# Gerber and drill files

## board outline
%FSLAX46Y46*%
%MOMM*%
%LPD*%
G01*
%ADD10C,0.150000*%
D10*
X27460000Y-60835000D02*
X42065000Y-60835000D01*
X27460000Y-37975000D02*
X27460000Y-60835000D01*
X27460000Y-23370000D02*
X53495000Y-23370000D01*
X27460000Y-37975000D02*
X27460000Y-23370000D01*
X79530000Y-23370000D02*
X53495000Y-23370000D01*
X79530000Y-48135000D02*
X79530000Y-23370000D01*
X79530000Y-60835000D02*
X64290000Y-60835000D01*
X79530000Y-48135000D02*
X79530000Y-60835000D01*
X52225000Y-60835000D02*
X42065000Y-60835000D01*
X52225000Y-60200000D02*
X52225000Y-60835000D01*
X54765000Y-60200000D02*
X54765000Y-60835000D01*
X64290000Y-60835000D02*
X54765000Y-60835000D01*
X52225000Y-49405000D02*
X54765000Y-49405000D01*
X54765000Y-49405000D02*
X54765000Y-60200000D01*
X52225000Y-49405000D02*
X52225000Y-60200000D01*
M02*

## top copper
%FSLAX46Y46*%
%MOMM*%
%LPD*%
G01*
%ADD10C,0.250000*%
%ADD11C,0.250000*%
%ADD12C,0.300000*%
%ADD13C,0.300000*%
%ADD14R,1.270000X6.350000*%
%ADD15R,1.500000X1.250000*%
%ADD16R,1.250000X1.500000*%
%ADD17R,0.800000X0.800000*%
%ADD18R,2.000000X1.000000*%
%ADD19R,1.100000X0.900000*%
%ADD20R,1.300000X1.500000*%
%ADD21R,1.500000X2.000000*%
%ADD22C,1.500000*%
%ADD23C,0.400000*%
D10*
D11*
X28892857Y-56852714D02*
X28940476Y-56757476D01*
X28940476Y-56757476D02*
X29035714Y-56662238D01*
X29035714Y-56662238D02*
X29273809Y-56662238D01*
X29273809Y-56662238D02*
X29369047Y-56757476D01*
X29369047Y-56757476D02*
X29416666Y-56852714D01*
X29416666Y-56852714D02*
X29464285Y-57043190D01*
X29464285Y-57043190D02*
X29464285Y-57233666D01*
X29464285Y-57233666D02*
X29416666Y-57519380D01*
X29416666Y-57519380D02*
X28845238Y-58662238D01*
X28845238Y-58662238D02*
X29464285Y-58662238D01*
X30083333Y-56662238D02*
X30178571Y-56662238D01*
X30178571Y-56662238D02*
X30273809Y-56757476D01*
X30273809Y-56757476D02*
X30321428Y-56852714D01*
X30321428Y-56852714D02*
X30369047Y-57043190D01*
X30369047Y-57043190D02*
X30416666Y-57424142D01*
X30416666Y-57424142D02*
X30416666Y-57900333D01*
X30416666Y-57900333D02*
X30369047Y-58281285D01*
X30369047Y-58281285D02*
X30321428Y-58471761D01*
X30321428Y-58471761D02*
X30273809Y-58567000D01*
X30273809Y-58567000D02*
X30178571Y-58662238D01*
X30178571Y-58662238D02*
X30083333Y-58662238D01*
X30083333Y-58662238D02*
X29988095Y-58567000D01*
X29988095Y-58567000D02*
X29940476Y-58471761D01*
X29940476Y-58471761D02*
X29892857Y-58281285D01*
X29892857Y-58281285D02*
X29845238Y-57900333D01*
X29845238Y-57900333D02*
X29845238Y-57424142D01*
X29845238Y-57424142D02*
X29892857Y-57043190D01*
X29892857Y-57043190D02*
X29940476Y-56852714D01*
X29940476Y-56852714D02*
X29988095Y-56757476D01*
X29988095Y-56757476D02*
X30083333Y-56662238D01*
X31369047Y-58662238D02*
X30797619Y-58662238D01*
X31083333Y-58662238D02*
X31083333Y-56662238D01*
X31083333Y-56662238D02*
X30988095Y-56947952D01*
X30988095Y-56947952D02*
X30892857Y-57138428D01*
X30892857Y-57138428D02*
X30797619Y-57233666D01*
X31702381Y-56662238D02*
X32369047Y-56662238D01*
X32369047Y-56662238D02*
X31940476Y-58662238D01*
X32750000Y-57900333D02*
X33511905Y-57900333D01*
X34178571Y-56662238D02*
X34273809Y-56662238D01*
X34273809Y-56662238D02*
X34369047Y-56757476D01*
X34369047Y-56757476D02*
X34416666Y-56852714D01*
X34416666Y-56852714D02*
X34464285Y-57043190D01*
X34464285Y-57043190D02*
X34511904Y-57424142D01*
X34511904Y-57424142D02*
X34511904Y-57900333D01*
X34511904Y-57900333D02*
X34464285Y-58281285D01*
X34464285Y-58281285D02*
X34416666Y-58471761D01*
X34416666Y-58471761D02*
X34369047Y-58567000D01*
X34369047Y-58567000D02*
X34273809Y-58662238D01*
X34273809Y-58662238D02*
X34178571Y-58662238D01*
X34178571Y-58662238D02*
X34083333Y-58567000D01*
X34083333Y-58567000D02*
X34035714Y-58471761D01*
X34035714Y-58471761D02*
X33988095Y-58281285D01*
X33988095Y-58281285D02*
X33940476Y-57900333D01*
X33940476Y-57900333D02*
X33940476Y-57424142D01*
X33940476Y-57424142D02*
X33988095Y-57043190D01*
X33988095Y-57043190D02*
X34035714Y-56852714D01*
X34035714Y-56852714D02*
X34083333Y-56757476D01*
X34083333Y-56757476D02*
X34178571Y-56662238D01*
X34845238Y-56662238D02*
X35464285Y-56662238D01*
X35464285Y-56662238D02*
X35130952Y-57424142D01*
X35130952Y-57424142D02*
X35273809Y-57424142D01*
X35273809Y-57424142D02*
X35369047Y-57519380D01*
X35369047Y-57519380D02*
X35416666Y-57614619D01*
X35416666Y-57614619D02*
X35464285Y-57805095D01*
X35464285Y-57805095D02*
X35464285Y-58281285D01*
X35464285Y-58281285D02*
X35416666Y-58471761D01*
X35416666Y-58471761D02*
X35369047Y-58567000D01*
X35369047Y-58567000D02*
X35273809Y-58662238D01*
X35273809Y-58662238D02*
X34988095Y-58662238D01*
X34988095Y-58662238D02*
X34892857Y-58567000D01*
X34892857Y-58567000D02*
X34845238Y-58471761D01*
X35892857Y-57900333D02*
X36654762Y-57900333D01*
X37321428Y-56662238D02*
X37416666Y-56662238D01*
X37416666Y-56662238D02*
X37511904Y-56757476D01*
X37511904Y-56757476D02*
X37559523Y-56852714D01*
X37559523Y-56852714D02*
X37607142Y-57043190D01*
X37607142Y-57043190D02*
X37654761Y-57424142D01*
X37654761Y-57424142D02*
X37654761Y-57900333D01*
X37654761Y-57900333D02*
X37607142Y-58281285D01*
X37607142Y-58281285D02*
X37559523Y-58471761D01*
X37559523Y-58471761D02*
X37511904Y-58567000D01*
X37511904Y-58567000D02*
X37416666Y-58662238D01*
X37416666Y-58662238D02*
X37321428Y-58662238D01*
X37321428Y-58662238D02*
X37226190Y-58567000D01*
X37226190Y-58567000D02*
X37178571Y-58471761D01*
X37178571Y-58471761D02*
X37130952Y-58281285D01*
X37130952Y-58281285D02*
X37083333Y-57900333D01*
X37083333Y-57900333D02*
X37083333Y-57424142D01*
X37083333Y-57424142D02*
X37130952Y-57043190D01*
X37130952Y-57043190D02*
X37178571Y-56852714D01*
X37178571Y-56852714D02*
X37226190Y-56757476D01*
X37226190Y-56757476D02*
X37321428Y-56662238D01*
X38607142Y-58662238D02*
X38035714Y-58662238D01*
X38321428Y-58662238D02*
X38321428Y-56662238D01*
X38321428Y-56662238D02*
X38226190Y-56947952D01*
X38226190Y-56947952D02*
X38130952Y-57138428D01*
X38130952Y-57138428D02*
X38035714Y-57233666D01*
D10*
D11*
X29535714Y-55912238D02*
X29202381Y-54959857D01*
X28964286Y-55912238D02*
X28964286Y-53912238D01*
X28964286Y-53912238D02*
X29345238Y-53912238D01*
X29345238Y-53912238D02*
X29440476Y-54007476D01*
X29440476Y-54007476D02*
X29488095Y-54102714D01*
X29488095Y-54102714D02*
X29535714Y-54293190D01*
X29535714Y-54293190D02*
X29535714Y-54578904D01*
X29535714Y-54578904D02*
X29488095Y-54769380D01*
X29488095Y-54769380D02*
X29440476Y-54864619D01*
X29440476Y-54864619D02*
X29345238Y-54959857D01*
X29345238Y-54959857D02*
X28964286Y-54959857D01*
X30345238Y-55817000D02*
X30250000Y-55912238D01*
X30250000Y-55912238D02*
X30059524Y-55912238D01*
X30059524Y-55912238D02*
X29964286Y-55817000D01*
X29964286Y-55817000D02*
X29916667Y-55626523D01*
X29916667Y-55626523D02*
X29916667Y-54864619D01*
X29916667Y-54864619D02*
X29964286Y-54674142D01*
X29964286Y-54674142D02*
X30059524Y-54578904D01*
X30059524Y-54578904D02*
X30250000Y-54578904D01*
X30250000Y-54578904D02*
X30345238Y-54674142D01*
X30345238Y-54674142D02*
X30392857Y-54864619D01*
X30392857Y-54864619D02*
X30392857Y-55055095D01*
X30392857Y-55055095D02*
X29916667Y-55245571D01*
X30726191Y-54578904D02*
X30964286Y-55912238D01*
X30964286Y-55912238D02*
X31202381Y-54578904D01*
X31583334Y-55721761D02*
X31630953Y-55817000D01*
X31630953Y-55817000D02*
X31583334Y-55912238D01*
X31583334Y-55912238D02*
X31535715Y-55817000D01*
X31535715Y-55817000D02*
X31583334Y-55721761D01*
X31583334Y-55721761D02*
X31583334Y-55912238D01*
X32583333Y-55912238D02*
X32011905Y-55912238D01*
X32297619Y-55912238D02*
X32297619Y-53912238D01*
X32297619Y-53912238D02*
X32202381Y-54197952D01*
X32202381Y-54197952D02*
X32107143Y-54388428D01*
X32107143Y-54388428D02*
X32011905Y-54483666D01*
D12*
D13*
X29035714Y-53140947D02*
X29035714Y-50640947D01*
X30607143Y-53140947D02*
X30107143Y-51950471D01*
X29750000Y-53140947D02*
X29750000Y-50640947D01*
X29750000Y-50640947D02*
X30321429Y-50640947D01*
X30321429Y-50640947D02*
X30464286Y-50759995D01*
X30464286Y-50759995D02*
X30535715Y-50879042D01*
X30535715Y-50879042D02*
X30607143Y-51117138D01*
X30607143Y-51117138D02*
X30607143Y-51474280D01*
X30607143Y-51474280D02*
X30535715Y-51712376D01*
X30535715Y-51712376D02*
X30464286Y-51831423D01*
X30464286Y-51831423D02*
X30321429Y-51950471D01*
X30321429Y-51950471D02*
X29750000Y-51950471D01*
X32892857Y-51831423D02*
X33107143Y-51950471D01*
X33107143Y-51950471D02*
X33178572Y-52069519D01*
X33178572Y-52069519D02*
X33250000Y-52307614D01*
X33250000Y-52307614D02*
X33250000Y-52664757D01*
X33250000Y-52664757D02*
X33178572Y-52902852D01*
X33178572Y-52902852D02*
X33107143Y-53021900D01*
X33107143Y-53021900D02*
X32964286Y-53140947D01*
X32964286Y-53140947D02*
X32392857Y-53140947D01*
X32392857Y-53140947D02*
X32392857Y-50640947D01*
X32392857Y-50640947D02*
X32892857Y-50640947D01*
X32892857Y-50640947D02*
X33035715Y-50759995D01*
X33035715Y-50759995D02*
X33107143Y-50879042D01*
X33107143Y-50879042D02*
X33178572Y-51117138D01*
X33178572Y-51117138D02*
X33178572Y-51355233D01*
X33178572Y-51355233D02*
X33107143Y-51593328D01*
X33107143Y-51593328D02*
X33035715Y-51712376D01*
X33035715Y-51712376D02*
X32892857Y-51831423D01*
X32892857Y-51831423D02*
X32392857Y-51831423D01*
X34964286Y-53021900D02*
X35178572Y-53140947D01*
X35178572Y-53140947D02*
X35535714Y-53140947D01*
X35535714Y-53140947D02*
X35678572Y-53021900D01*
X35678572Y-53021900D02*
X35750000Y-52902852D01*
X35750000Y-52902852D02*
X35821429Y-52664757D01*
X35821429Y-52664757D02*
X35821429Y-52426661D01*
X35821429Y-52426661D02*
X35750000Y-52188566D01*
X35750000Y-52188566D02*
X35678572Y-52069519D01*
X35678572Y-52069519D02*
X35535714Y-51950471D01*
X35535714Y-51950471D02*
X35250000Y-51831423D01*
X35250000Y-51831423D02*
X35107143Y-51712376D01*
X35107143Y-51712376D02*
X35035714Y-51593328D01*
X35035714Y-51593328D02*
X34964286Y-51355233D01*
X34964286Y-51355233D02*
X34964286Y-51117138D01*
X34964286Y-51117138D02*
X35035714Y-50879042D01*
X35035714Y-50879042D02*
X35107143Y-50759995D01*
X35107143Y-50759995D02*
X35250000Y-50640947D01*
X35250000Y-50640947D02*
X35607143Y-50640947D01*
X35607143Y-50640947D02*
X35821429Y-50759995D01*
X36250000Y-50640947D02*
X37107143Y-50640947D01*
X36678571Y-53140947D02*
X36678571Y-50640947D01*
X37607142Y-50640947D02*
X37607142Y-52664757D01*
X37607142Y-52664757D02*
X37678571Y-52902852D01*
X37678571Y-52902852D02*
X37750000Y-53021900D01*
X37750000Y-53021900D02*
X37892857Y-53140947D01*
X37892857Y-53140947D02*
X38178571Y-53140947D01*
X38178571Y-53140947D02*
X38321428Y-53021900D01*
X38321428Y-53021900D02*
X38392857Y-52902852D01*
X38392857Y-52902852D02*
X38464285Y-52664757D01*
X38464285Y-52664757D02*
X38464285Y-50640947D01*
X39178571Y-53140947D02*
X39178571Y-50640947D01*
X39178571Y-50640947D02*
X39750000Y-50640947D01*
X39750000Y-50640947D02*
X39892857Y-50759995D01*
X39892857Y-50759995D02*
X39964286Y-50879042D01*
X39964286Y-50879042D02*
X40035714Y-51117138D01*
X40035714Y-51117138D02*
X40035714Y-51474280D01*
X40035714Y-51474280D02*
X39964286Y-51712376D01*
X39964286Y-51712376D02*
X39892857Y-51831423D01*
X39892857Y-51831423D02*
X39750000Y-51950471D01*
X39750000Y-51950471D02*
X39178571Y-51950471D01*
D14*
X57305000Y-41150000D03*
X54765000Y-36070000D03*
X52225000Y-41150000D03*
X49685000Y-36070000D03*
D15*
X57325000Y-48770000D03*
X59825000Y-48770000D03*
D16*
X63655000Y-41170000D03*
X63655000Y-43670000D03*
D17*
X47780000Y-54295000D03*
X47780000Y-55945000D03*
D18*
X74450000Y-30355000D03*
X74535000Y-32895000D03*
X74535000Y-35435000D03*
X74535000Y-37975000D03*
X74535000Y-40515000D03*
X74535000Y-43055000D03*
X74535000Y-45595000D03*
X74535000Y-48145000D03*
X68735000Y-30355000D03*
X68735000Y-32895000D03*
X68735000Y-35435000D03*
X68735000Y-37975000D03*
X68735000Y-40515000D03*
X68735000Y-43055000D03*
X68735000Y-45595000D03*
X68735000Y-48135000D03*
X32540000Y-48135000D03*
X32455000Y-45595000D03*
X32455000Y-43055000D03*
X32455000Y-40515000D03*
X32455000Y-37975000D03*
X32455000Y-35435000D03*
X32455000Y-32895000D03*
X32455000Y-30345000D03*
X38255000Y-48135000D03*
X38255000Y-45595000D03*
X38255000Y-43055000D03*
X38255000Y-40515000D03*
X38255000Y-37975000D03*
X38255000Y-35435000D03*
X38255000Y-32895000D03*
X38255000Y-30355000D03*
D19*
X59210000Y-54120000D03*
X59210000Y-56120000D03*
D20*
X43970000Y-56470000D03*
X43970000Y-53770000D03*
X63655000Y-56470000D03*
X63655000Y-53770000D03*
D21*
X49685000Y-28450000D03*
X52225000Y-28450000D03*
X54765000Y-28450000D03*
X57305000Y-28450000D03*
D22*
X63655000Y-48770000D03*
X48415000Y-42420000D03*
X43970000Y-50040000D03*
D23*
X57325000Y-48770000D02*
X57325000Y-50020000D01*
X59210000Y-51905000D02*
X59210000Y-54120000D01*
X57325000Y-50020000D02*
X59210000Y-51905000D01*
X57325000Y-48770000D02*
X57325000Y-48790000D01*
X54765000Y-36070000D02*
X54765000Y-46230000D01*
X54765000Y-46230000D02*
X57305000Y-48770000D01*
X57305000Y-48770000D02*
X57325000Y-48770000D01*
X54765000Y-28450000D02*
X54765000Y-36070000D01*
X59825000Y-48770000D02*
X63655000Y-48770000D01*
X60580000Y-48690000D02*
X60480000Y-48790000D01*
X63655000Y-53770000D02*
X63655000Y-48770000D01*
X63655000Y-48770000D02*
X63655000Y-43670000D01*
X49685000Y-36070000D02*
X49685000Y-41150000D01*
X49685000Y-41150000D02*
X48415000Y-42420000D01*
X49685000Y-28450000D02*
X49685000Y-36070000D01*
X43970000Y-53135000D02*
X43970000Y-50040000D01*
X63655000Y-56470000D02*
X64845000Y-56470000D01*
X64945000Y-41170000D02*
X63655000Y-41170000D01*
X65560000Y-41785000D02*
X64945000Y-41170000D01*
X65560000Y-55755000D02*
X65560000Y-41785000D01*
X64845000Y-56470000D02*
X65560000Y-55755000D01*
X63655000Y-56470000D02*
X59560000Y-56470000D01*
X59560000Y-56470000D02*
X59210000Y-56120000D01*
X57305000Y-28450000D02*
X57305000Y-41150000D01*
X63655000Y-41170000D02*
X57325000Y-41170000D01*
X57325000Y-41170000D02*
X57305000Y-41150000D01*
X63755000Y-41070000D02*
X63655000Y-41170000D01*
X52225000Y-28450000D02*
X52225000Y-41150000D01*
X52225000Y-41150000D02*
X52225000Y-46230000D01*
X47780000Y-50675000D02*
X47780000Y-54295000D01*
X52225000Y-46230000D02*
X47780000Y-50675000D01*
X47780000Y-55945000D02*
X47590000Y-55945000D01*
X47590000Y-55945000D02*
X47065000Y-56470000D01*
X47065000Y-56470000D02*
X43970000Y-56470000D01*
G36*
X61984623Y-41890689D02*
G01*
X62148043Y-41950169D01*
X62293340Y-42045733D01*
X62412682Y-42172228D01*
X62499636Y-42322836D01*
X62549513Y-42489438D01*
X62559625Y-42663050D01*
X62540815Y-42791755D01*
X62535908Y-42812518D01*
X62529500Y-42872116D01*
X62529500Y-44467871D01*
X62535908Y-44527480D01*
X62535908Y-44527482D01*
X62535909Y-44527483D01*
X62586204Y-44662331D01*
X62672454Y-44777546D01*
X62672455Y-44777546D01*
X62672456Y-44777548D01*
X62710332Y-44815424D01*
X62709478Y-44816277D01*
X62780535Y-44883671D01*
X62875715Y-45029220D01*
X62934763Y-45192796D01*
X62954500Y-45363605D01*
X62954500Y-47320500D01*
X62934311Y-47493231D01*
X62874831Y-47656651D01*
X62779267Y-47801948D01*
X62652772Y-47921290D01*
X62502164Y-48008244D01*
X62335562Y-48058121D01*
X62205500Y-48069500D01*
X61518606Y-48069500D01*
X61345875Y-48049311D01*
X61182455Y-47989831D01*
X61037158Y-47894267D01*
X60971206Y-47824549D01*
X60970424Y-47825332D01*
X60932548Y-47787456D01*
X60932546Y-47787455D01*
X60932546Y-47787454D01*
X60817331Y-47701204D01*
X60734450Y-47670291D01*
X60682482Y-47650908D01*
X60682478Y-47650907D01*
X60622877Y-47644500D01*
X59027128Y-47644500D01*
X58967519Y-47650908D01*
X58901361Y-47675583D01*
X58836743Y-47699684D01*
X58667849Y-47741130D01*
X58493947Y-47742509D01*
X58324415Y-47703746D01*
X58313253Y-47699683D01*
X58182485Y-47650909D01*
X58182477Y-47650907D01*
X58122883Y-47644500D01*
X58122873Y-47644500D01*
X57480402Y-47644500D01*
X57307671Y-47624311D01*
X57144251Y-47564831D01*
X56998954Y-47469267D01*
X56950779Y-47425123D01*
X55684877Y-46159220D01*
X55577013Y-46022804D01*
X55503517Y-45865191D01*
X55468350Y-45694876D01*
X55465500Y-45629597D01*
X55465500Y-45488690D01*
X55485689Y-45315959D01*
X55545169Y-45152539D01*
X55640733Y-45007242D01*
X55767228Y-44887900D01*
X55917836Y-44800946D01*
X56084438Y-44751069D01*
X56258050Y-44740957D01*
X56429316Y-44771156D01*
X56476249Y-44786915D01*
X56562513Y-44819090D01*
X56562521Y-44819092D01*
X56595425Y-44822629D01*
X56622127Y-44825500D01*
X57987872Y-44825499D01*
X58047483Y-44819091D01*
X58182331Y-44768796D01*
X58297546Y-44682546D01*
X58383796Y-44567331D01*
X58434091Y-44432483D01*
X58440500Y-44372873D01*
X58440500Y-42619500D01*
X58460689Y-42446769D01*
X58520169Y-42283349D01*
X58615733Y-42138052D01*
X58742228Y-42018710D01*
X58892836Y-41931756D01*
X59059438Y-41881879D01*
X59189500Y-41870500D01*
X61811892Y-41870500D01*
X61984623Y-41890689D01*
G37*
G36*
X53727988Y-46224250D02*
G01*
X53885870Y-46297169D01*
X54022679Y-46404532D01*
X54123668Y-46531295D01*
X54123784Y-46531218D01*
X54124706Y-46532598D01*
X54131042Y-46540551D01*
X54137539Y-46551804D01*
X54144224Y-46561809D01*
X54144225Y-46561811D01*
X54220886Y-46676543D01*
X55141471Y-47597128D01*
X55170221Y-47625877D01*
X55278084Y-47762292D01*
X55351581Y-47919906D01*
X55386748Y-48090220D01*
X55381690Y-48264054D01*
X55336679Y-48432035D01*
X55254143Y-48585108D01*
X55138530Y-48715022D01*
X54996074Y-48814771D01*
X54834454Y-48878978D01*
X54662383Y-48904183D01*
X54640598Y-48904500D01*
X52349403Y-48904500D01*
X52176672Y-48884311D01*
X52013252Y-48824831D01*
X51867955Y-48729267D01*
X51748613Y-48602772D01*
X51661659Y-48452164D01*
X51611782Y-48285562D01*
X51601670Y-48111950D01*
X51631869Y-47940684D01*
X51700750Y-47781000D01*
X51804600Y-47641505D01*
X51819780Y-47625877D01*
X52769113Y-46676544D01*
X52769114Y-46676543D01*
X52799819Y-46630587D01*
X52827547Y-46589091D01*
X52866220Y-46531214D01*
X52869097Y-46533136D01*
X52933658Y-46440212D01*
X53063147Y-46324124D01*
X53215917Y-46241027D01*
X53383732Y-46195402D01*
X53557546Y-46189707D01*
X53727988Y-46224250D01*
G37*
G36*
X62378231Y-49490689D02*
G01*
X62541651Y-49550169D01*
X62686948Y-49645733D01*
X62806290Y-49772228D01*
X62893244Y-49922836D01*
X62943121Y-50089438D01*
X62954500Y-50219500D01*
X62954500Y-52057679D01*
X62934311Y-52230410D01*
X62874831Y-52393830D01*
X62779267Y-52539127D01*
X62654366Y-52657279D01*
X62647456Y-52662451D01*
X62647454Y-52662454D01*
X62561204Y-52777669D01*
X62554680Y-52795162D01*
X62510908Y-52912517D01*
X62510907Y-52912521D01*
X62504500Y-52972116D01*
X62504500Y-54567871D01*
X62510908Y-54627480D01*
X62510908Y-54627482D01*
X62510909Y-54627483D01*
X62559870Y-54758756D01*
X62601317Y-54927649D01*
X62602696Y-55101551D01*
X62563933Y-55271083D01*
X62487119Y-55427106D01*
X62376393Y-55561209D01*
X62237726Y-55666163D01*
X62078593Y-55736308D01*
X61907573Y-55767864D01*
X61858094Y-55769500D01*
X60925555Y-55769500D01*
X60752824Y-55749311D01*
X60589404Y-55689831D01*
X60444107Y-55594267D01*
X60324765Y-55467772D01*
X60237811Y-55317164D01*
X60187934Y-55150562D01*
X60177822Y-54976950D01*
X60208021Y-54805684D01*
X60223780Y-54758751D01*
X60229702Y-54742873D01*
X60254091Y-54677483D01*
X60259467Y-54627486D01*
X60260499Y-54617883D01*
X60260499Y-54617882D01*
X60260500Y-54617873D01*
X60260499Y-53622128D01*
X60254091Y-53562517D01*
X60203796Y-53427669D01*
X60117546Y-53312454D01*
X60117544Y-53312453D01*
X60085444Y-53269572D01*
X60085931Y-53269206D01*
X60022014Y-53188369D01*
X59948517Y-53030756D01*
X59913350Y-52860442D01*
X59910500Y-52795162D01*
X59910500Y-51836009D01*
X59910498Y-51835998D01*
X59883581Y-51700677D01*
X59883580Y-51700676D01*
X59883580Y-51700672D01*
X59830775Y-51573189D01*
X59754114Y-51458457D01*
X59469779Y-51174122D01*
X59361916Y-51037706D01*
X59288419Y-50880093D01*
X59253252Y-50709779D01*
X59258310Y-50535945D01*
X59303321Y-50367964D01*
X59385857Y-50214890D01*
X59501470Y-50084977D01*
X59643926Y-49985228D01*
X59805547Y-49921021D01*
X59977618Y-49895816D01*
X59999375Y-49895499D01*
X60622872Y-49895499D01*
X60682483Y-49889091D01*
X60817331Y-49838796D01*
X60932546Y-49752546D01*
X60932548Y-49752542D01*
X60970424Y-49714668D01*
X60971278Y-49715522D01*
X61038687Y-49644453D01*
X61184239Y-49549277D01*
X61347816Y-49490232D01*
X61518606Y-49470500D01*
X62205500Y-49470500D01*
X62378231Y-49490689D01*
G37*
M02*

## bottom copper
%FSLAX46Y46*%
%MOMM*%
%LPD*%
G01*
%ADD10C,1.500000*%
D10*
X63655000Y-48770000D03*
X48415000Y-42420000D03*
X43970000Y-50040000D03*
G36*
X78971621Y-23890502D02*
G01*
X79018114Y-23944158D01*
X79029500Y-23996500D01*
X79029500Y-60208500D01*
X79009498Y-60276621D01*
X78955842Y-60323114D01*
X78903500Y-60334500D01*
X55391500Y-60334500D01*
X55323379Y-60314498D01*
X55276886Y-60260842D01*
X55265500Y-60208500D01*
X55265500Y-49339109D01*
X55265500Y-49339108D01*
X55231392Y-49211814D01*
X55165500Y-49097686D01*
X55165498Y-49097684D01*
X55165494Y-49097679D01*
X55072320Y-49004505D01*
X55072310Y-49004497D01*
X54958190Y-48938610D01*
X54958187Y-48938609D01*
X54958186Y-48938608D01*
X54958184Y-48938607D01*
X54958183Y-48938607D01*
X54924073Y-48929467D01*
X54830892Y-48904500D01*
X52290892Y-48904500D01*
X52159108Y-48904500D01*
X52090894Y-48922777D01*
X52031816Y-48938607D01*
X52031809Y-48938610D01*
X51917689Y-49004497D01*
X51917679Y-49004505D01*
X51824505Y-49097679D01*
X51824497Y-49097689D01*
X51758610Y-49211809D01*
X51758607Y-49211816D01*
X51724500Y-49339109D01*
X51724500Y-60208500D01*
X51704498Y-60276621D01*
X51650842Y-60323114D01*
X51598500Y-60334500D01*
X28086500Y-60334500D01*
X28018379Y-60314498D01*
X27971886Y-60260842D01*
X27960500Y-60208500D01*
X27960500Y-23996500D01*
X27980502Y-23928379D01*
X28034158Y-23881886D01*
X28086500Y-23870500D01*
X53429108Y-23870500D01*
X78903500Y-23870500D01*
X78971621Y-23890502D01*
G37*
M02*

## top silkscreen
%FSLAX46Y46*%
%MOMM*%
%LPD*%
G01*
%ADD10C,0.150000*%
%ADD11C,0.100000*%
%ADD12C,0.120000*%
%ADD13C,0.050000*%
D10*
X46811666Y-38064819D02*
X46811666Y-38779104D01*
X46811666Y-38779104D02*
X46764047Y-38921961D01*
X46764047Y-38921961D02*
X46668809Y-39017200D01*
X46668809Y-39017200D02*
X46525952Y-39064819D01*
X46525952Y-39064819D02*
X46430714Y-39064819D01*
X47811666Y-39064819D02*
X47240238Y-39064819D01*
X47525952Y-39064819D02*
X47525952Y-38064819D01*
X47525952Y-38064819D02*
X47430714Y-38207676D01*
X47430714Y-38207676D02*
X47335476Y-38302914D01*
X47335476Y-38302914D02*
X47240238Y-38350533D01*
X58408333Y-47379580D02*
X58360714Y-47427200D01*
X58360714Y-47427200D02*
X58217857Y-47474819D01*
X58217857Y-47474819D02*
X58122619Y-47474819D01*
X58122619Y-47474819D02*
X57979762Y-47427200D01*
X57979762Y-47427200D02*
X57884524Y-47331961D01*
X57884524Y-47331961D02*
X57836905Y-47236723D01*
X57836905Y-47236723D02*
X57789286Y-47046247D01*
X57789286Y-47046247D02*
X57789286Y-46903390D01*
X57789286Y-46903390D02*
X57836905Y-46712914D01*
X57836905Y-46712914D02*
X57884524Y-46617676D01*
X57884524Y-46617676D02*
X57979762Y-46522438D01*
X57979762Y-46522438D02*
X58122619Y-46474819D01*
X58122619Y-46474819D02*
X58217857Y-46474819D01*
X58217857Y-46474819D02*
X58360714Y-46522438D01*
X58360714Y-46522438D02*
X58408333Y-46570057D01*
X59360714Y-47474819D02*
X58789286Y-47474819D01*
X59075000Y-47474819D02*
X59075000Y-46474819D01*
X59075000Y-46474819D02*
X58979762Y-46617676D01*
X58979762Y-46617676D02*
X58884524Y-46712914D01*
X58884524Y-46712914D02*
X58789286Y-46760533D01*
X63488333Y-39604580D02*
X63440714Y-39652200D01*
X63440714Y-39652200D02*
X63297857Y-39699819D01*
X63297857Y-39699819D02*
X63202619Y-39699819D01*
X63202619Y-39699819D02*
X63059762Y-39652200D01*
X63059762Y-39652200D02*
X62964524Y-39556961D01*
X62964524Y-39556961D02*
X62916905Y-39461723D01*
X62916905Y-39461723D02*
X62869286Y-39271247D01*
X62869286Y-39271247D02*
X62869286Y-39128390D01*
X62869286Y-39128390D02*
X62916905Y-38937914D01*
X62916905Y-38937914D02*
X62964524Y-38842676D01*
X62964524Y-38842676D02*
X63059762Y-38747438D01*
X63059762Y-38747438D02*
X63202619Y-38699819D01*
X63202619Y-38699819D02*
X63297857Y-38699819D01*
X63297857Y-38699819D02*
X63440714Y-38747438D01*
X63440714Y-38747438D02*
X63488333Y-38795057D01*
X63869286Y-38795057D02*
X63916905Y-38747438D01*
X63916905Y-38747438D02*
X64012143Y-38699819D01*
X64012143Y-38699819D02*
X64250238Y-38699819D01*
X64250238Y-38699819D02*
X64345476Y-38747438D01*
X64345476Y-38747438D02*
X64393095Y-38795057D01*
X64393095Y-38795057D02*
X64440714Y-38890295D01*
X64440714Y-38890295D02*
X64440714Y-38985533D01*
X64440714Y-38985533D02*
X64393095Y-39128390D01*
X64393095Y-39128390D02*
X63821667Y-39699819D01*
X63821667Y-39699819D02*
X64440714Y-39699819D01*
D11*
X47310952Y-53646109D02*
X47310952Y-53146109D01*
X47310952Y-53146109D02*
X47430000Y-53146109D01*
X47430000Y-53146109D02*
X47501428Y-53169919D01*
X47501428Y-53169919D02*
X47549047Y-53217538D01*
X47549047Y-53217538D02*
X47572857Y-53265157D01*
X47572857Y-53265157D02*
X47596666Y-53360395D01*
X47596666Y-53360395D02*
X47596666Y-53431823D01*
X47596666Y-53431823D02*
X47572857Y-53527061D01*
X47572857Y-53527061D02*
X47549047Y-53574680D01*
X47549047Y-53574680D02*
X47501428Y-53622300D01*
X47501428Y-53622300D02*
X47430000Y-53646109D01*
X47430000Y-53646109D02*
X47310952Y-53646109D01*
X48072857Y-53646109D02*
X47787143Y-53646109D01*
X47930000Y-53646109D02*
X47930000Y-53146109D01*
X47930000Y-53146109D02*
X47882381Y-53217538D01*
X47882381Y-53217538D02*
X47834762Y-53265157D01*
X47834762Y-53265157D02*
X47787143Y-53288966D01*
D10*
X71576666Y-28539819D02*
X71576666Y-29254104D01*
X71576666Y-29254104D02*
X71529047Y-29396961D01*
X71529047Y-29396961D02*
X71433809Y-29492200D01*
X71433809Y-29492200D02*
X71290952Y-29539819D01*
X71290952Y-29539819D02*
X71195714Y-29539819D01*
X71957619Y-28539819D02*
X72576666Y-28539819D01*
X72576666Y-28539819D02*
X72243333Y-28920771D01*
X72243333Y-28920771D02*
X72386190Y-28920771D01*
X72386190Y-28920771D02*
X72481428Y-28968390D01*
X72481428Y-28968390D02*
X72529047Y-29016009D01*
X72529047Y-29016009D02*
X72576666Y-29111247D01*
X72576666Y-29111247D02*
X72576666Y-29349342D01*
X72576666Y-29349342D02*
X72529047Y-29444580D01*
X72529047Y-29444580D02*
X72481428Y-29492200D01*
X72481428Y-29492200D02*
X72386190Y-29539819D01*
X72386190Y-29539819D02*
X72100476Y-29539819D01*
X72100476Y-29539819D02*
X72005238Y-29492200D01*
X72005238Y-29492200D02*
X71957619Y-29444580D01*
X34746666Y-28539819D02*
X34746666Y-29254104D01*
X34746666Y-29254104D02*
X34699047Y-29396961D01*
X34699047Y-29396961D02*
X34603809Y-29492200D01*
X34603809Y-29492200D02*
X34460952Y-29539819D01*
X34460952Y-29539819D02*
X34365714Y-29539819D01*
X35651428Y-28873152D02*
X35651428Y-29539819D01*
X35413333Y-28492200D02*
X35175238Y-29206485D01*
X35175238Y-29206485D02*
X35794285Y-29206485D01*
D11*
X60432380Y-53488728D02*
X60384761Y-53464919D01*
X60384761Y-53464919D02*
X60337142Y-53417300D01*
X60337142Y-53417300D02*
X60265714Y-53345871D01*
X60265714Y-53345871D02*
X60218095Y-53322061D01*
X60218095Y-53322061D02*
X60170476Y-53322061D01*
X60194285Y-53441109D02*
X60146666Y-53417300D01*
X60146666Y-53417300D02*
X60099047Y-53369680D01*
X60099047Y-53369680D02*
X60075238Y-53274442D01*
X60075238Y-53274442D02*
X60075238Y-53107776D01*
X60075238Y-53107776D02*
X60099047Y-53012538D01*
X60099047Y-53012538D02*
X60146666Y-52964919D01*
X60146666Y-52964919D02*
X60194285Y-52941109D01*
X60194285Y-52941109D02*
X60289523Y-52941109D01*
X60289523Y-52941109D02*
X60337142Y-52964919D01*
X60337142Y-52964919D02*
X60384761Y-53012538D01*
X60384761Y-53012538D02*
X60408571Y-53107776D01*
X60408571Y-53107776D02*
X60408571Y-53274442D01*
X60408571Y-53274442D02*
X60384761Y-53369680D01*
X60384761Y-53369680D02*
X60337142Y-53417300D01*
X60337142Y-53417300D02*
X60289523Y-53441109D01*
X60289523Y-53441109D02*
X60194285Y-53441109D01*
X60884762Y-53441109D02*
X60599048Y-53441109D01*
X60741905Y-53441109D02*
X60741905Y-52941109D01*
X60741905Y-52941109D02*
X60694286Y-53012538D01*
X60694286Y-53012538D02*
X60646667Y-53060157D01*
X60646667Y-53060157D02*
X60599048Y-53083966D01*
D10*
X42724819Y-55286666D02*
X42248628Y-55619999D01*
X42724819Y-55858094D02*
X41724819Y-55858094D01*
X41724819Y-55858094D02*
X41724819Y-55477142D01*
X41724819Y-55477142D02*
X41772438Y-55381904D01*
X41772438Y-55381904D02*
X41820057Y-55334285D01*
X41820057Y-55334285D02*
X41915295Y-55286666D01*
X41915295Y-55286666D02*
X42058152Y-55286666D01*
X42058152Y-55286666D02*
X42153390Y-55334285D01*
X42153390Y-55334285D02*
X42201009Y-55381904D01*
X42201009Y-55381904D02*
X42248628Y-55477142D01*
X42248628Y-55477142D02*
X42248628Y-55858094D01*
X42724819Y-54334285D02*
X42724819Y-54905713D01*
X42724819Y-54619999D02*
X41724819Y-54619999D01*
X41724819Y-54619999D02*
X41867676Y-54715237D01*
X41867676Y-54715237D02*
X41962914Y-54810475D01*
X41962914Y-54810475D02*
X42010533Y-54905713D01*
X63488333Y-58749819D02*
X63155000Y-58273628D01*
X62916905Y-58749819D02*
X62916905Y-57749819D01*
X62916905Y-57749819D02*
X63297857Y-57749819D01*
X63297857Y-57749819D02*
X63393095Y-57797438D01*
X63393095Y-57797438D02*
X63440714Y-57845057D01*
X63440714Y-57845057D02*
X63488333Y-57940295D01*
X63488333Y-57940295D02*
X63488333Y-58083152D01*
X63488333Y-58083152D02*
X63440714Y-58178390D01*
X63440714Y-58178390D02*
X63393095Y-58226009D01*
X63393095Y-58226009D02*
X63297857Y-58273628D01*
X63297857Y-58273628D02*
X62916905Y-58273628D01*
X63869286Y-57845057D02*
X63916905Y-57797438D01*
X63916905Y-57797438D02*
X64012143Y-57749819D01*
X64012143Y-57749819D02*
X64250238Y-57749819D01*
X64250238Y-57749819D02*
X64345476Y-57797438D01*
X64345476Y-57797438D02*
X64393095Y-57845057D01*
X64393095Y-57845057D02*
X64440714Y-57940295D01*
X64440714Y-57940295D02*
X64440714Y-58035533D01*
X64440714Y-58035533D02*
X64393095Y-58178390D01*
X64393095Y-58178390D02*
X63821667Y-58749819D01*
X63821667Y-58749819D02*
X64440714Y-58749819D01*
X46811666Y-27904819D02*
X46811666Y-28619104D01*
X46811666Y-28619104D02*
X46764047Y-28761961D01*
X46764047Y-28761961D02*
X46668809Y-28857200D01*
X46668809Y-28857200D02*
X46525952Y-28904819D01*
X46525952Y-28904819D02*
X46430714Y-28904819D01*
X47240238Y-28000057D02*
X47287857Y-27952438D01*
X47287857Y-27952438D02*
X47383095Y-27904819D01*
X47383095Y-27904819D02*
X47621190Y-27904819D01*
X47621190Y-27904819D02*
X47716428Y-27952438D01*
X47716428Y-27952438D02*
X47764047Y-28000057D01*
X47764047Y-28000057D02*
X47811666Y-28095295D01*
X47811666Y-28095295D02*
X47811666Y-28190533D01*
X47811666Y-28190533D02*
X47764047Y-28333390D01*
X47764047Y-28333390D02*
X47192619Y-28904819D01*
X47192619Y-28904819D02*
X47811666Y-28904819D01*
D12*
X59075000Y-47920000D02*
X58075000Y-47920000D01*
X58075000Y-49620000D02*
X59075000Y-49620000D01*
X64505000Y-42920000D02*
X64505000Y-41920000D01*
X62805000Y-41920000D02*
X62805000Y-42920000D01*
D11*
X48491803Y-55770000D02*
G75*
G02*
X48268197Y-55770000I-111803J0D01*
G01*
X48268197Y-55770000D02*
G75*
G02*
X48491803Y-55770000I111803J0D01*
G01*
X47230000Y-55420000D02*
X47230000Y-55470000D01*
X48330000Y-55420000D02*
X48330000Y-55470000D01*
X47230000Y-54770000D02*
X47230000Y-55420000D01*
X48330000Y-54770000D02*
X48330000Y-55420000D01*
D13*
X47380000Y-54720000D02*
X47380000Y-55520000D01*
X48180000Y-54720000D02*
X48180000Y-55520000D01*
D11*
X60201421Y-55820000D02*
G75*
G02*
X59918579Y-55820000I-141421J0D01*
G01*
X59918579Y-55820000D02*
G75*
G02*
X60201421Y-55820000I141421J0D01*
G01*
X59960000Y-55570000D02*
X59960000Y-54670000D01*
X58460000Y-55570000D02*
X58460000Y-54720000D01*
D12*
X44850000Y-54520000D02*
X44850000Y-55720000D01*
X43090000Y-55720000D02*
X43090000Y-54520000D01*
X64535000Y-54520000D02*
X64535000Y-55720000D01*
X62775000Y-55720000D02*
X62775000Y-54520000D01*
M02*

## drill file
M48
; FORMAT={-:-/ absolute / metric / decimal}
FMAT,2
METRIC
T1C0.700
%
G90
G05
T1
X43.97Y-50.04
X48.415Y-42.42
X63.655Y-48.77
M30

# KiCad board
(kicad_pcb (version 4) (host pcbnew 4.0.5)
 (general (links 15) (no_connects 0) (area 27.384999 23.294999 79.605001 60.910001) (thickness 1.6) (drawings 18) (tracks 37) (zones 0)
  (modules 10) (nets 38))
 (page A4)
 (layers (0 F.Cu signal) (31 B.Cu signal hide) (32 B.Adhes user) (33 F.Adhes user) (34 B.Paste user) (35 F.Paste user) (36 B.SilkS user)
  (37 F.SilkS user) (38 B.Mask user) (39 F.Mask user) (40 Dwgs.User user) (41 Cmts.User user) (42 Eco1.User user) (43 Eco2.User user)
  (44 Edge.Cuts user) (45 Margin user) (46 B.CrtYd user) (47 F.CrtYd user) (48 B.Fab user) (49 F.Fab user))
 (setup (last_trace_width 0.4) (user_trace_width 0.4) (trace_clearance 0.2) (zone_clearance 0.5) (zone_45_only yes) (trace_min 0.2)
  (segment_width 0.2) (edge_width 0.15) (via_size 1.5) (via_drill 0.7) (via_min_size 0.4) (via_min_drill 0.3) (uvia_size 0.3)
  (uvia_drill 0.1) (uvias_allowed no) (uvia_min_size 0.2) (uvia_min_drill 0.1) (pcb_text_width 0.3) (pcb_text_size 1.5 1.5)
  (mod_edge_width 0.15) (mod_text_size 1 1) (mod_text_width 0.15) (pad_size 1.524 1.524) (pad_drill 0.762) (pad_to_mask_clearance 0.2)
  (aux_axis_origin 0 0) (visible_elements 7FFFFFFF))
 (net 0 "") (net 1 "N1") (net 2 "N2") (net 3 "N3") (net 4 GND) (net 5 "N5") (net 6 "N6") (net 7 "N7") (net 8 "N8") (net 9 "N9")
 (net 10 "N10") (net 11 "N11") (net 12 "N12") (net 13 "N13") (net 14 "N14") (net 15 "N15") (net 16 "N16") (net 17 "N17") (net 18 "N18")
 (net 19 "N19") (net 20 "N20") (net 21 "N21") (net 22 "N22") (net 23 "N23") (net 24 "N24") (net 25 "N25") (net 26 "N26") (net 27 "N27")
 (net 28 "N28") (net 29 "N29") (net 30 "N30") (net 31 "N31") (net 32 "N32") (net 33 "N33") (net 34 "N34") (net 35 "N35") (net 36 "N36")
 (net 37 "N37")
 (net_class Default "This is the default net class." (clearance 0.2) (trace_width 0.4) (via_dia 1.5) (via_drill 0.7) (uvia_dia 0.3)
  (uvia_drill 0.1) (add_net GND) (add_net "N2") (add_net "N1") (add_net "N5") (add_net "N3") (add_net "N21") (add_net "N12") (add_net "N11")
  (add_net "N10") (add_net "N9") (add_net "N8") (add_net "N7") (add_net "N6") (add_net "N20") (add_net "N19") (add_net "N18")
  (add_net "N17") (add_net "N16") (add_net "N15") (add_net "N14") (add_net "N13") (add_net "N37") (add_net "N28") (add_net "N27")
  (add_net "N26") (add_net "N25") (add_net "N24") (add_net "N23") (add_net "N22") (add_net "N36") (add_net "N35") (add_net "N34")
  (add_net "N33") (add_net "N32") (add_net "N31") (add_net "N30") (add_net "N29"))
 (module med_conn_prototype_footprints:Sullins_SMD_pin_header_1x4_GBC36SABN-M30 (layer F.Cu) (at 53.495 30.99)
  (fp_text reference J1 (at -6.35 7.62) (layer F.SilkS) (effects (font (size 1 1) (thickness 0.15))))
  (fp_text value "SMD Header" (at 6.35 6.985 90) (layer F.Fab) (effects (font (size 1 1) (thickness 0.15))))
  (pad 4 smd rect (at 3.81 10.16) (size 1.27 6.35) (layers F.Cu F.Paste F.Mask) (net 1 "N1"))
  (pad 3 smd rect (at 1.27 5.08) (size 1.27 6.35) (layers F.Cu F.Paste F.Mask) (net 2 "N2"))
  (pad 2 smd rect (at -1.27 10.16) (size 1.27 6.35) (layers F.Cu F.Paste F.Mask) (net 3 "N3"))
  (pad 1 smd rect (at -3.81 5.08) (size 1.27 6.35) (layers F.Cu F.Paste F.Mask) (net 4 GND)))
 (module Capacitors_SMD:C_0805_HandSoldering (layer F.Cu) (at 58.575 48.77)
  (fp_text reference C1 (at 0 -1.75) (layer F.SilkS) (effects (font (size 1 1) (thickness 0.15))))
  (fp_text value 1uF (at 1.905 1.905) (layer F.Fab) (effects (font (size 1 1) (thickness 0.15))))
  (fp_line (start 0.5 -0.85) (end -0.5 -0.85) (layer F.SilkS) (width 0.12))
  (fp_line (start -0.5 0.85) (end 0.5 0.85) (layer F.SilkS) (width 0.12))
  (pad 1 smd rect (at -1.25 0) (size 1.5 1.25) (layers F.Cu F.Paste F.Mask) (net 2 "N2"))
  (pad 2 smd rect (at 1.25 0) (size 1.5 1.25) (layers F.Cu F.Paste F.Mask) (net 4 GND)))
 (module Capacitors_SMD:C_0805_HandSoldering (layer F.Cu) (at 63.655 42.42 270)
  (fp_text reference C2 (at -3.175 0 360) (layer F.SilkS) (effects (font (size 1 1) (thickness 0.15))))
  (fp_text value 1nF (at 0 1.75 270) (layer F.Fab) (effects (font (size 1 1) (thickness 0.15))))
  (fp_line (start 0.5 -0.85) (end -0.5 -0.85) (layer F.SilkS) (width 0.12))
  (fp_line (start -0.5 0.85) (end 0.5 0.85) (layer F.SilkS) (width 0.12))
  (pad 1 smd rect (at -1.25 0 270) (size 1.5 1.25) (layers F.Cu F.Paste F.Mask) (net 1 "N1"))
  (pad 2 smd rect (at 1.25 0 270) (size 1.5 1.25) (layers F.Cu F.Paste F.Mask) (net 4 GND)))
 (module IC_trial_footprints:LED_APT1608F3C (layer F.Cu) (at 47.78 55.12 270)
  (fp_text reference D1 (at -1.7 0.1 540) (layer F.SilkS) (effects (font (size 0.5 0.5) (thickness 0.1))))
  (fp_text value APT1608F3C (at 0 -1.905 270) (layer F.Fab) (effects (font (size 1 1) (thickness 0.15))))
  (fp_circle (center 0.65 -0.6) (end 0.7 -0.7) (layer F.SilkS) (width 0.1))
  (fp_line (start 0.3 0.55) (end 0.35 0.55) (layer F.SilkS) (width 0.1))
  (fp_line (start 0.3 -0.55) (end 0.35 -0.55) (layer F.SilkS) (width 0.1))
  (fp_line (start -0.35 0.55) (end 0.3 0.55) (layer F.SilkS) (width 0.1))
  (fp_line (start -0.35 -0.55) (end 0.3 -0.55) (layer F.SilkS) (width 0.1))
  (fp_line (start -0.4 0.4) (end 0.4 0.4) (layer F.SilkS) (width 0.05))
  (fp_line (start -0.4 -0.4) (end 0.4 -0.4) (layer F.SilkS) (width 0.05))
  (pad 2 smd rect (at -0.825 0 270) (size 0.8 0.8) (layers F.Cu F.Paste F.Mask) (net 3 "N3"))
  (pad 1 smd rect (at 0.825 0 270) (size 0.8 0.8) (layers F.Cu F.Paste F.Mask) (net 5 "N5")))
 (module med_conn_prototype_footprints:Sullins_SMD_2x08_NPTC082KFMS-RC (layer F.Cu) (at 64.925 39.245 90)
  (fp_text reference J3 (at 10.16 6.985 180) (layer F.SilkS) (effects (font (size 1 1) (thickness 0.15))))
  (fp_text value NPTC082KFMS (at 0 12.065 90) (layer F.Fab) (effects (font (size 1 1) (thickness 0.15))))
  (pad 16 smd rect (at 8.89 9.525 90) (size 1 2) (layers F.Cu F.Paste F.Mask) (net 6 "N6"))
  (pad 15 smd rect (at 6.35 9.61 90) (size 1 2) (layers F.Cu F.Paste F.Mask) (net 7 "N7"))
  (pad 14 smd rect (at 3.81 9.61 90) (size 1 2) (layers F.Cu F.Paste F.Mask) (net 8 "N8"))
  (pad 13 smd rect (at 1.27 9.61 90) (size 1 2) (layers F.Cu F.Paste F.Mask) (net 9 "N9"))
  (pad 12 smd rect (at -1.27 9.61 90) (size 1 2) (layers F.Cu F.Paste F.Mask) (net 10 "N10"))
  (pad 11 smd rect (at -3.81 9.61 90) (size 1 2) (layers F.Cu F.Paste F.Mask) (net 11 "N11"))
  (pad 10 smd rect (at -6.35 9.61 90) (size 1 2) (layers F.Cu F.Paste F.Mask) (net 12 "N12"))
  (pad 9 smd rect (at -8.9 9.61 90) (size 1 2) (layers F.Cu F.Paste F.Mask) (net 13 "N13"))
  (pad 8 smd rect (at 8.89 3.81 90) (size 1 2) (layers F.Cu F.Paste F.Mask) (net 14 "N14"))
  (pad 7 smd rect (at 6.35 3.81 90) (size 1 2) (layers F.Cu F.Paste F.Mask) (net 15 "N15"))
  (pad 6 smd rect (at 3.81 3.81 90) (size 1 2) (layers F.Cu F.Paste F.Mask) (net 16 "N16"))
  (pad 5 smd rect (at 1.27 3.81 90) (size 1 2) (layers F.Cu F.Paste F.Mask) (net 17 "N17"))
  (pad 4 smd rect (at -1.27 3.81 90) (size 1 2) (layers F.Cu F.Paste F.Mask) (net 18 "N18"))
  (pad 3 smd rect (at -3.81 3.81 90) (size 1 2) (layers F.Cu F.Paste F.Mask) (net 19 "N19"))
  (pad 2 smd rect (at -6.35 3.81 90) (size 1 2) (layers F.Cu F.Paste F.Mask) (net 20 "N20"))
  (pad 1 smd rect (at -8.89 3.81 90) (size 1 2) (layers F.Cu F.Paste F.Mask) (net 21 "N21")))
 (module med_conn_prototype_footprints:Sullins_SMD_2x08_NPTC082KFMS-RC (layer F.Cu) (at 42.065 39.245 270)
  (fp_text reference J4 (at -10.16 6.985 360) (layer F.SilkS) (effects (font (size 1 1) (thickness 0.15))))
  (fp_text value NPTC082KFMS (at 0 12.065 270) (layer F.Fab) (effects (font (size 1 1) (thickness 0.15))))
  (pad 16 smd rect (at 8.89 9.525 270) (size 1 2) (layers F.Cu F.Paste F.Mask) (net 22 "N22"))
  (pad 15 smd rect (at 6.35 9.61 270) (size 1 2) (layers F.Cu F.Paste F.Mask) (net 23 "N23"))
  (pad 14 smd rect (at 3.81 9.61 270) (size 1 2) (layers F.Cu F.Paste F.Mask) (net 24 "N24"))
  (pad 13 smd rect (at 1.27 9.61 270) (size 1 2) (layers F.Cu F.Paste F.Mask) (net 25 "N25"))
  (pad 12 smd rect (at -1.27 9.61 270) (size 1 2) (layers F.Cu F.Paste F.Mask) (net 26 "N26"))
  (pad 11 smd rect (at -3.81 9.61 270) (size 1 2) (layers F.Cu F.Paste F.Mask) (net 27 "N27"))
  (pad 10 smd rect (at -6.35 9.61 270) (size 1 2) (layers F.Cu F.Paste F.Mask) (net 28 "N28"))
  (pad 9 smd rect (at -8.9 9.61 270) (size 1 2) (layers F.Cu F.Paste F.Mask) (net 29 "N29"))
  (pad 8 smd rect (at 8.89 3.81 270) (size 1 2) (layers F.Cu F.Paste F.Mask) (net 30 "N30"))
  (pad 7 smd rect (at 6.35 3.81 270) (size 1 2) (layers F.Cu F.Paste F.Mask) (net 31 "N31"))
  (pad 6 smd rect (at 3.81 3.81 270) (size 1 2) (layers F.Cu F.Paste F.Mask) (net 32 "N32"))
  (pad 5 smd rect (at 1.27 3.81 270) (size 1 2) (layers F.Cu F.Paste F.Mask) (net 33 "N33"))
  (pad 4 smd rect (at -1.27 3.81 270) (size 1 2) (layers F.Cu F.Paste F.Mask) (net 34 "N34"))
  (pad 3 smd rect (at -3.81 3.81 270) (size 1 2) (layers F.Cu F.Paste F.Mask) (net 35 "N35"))
  (pad 2 smd rect (at -6.35 3.81 270) (size 1 2) (layers F.Cu F.Paste F.Mask) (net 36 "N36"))
  (pad 1 smd rect (at -8.89 3.81 270) (size 1 2) (layers F.Cu F.Paste F.Mask) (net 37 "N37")))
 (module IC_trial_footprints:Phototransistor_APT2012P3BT (layer F.Cu) (at 59.21 55.12 90)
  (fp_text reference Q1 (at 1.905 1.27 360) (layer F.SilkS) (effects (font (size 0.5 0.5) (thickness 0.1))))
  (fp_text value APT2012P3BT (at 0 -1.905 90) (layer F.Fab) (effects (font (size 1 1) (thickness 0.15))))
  (fp_circle (center -0.7 0.85) (end -0.6 0.95) (layer F.SilkS) (width 0.1))
  (fp_line (start -0.45 0.75) (end 0.45 0.75) (layer F.SilkS) (width 0.1))
  (fp_line (start -0.45 -0.75) (end 0.4 -0.75) (layer F.SilkS) (width 0.1))
  (pad 2 smd rect (at 1 0 90) (size 0.9 1.1) (layers F.Cu F.Paste F.Mask) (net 2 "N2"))
  (pad 1 smd rect (at -1 0 90) (size 0.9 1.1) (layers F.Cu F.Paste F.Mask) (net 1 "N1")))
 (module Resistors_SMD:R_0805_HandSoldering (layer F.Cu) (at 43.97 55.12 90)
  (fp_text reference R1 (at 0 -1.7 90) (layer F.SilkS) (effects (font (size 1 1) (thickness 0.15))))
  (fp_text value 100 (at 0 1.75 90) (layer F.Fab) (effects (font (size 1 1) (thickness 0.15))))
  (fp_line (start 0.6 0.88) (end -0.6 0.88) (layer F.SilkS) (width 0.12))
  (fp_line (start -0.6 -0.88) (end 0.6 -0.88) (layer F.SilkS) (width 0.12))
  (pad 1 smd rect (at -1.35 0 90) (size 1.5 1.3) (layers F.Cu F.Paste F.Mask) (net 5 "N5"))
  (pad 2 smd rect (at 1.35 0 90) (size 1.5 1.3) (layers F.Cu F.Paste F.Mask) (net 4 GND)))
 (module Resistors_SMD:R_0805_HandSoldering (layer F.Cu) (at 63.655 55.12 90)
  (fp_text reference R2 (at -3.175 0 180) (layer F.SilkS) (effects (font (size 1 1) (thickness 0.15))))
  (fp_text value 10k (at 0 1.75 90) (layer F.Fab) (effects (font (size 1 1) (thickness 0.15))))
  (fp_line (start 0.6 0.88) (end -0.6 0.88) (layer F.SilkS) (width 0.12))
  (fp_line (start -0.6 -0.88) (end 0.6 -0.88) (layer F.SilkS) (width 0.12))
  (pad 1 smd rect (at -1.35 0 90) (size 1.5 1.3) (layers F.Cu F.Paste F.Mask) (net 1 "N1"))
  (pad 2 smd rect (at 1.35 0 90) (size 1.5 1.3) (layers F.Cu F.Paste F.Mask) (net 4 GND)))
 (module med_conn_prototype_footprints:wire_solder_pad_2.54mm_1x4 (layer F.Cu) (at 53.495 24.64)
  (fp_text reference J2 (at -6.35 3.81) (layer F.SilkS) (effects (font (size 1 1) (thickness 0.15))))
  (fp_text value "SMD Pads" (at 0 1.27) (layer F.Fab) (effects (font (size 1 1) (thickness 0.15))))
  (pad 1 smd rect (at -3.81 3.81) (size 1.5 2) (layers F.Cu F.Paste F.Mask) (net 4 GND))
  (pad 2 smd rect (at -1.27 3.81) (size 1.5 2) (layers F.Cu F.Paste F.Mask) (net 3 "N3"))
  (pad 3 smd rect (at 1.27 3.81) (size 1.5 2) (layers F.Cu F.Paste F.Mask) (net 2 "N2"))
  (pad 4 smd rect (at 3.81 3.81) (size 1.5 2) (layers F.Cu F.Paste F.Mask) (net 1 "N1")))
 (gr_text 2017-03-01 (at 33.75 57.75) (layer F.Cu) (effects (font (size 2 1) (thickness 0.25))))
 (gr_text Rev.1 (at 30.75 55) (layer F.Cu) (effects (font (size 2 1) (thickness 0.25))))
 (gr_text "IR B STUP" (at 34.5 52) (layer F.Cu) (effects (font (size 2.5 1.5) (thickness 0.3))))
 (gr_line (start 27.46 60.835) (end 42.065 60.835) (angle 90) (layer Edge.Cuts) (width 0.15))
 (gr_line (start 27.46 37.975) (end 27.46 60.835) (angle 90) (layer Edge.Cuts) (width 0.15))
 (gr_line (start 27.46 23.37) (end 53.495 23.37) (angle 90) (layer Edge.Cuts) (width 0.15))
 (gr_line (start 27.46 37.975) (end 27.46 23.37) (angle 90) (layer Edge.Cuts) (width 0.15))
 (gr_line (start 79.53 23.37) (end 53.495 23.37) (angle 90) (layer Edge.Cuts) (width 0.15))
 (gr_line (start 79.53 48.135) (end 79.53 23.37) (angle 90) (layer Edge.Cuts) (width 0.15))
 (gr_line (start 79.53 60.835) (end 64.29 60.835) (angle 90) (layer Edge.Cuts) (width 0.15))
 (gr_line (start 79.53 48.135) (end 79.53 60.835) (angle 90) (layer Edge.Cuts) (width 0.15))
 (gr_line (start 52.225 60.835) (end 42.065 60.835) (angle 90) (layer Edge.Cuts) (width 0.15))
 (gr_line (start 52.225 60.2) (end 52.225 60.835) (angle 90) (layer Edge.Cuts) (width 0.15))
 (gr_line (start 54.765 60.2) (end 54.765 60.835) (angle 90) (layer Edge.Cuts) (width 0.15))
 (gr_line (start 64.29 60.835) (end 54.765 60.835) (angle 90) (layer Edge.Cuts) (width 0.15))
 (gr_line (start 52.225 49.405) (end 54.765 49.405) (angle 90) (layer Edge.Cuts) (width 0.15))
 (gr_line (start 54.765 49.405) (end 54.765 60.2) (angle 90) (layer Edge.Cuts) (width 0.15))
 (gr_line (start 52.225 49.405) (end 52.225 60.2) (angle 90) (layer Edge.Cuts) (width 0.15))
 (segment (start 57.325 48.77) (end 57.325 50.02) (width 0.4) (layer F.Cu) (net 2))
 (segment (start 59.21 51.905) (end 59.21 54.12) (width 0.4) (layer F.Cu) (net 2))
 (segment (start 57.325 50.02) (end 59.21 51.905) (width 0.4) (layer F.Cu) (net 2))
 (segment (start 57.325 48.77) (end 57.325 48.79) (width 0.4) (layer F.Cu) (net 2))
 (segment (start 54.765 36.07) (end 54.765 46.23) (width 0.4) (layer F.Cu) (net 2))
 (segment (start 54.765 46.23) (end 57.305 48.77) (width 0.4) (layer F.Cu) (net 2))
 (segment (start 57.305 48.77) (end 57.325 48.77) (width 0.4) (layer F.Cu) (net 2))
 (segment (start 54.765 28.45) (end 54.765 36.07) (width 0.4) (layer F.Cu) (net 2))
 (segment (start 59.825 48.77) (end 63.655 48.77) (width 0.4) (layer F.Cu) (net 4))
 (via (at 63.655 48.77) (size 1.5) (drill 0.7) (layers F.Cu B.Cu) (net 4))
 (segment (start 60.58 48.69) (end 60.48 48.79) (width 0.4) (layer F.Cu) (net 4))
 (segment (start 63.655 53.77) (end 63.655 48.77) (width 0.4) (layer F.Cu) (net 4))
 (segment (start 63.655 48.77) (end 63.655 43.67) (width 0.4) (layer F.Cu) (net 4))
 (segment (start 49.685 36.07) (end 49.685 41.15) (width 0.4) (layer F.Cu) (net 4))
 (via (at 48.415 42.42) (size 1.5) (drill 0.7) (layers F.Cu B.Cu) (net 4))
 (segment (start 49.685 41.15) (end 48.415 42.42) (width 0.4) (layer F.Cu) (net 4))
 (segment (start 49.685 28.45) (end 49.685 36.07) (width 0.4) (layer F.Cu) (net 4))
 (segment (start 43.97 53.135) (end 43.97 50.04) (width 0.4) (layer F.Cu) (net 4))
 (via (at 43.97 50.04) (size 1.5) (drill 0.7) (layers F.Cu B.Cu) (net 4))
 (segment (start 63.655 56.47) (end 64.845 56.47) (width 0.4) (layer F.Cu) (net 1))
 (segment (start 64.945 41.17) (end 63.655 41.17) (width 0.4) (layer F.Cu) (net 1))
 (segment (start 65.56 41.785) (end 64.945 41.17) (width 0.4) (layer F.Cu) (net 1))
 (segment (start 65.56 55.755) (end 65.56 41.785) (width 0.4) (layer F.Cu) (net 1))
 (segment (start 64.845 56.47) (end 65.56 55.755) (width 0.4) (layer F.Cu) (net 1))
 (segment (start 63.655 56.47) (end 59.56 56.47) (width 0.4) (layer F.Cu) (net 1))
 (segment (start 59.56 56.47) (end 59.21 56.12) (width 0.4) (layer F.Cu) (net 1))
 (segment (start 57.305 28.45) (end 57.305 41.15) (width 0.4) (layer F.Cu) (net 1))
 (segment (start 63.655 41.17) (end 57.325 41.17) (width 0.4) (layer F.Cu) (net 1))
 (segment (start 57.325 41.17) (end 57.305 41.15) (width 0.4) (layer F.Cu) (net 1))
 (segment (start 63.755 41.07) (end 63.655 41.17) (width 0.4) (layer F.Cu) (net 1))
 (segment (start 52.225 28.45) (end 52.225 41.15) (width 0.4) (layer F.Cu) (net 3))
 (segment (start 52.225 41.15) (end 52.225 46.23) (width 0.4) (layer F.Cu) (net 3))
 (segment (start 47.78 50.675) (end 47.78 54.295) (width 0.4) (layer F.Cu) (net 3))
 (segment (start 52.225 46.23) (end 47.78 50.675) (width 0.4) (layer F.Cu) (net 3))
 (segment (start 47.78 55.945) (end 47.59 55.945) (width 0.4) (layer F.Cu) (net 5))
 (segment (start 47.59 55.945) (end 47.065 56.47) (width 0.4) (layer F.Cu) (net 5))
 (segment (start 47.065 56.47) (end 43.97 56.47) (width 0.4) (layer F.Cu) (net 5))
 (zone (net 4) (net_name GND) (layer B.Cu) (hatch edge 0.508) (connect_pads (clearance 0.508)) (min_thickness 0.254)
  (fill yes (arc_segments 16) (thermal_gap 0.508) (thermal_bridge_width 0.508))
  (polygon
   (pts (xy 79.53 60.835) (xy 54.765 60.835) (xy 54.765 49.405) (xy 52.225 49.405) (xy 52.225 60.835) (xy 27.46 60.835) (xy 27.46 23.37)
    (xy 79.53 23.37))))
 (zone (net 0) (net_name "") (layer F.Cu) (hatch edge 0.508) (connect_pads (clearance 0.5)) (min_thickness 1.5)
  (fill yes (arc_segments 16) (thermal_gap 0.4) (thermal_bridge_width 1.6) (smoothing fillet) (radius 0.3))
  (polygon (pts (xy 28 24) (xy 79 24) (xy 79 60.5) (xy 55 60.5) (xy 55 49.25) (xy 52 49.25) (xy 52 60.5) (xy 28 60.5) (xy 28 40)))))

